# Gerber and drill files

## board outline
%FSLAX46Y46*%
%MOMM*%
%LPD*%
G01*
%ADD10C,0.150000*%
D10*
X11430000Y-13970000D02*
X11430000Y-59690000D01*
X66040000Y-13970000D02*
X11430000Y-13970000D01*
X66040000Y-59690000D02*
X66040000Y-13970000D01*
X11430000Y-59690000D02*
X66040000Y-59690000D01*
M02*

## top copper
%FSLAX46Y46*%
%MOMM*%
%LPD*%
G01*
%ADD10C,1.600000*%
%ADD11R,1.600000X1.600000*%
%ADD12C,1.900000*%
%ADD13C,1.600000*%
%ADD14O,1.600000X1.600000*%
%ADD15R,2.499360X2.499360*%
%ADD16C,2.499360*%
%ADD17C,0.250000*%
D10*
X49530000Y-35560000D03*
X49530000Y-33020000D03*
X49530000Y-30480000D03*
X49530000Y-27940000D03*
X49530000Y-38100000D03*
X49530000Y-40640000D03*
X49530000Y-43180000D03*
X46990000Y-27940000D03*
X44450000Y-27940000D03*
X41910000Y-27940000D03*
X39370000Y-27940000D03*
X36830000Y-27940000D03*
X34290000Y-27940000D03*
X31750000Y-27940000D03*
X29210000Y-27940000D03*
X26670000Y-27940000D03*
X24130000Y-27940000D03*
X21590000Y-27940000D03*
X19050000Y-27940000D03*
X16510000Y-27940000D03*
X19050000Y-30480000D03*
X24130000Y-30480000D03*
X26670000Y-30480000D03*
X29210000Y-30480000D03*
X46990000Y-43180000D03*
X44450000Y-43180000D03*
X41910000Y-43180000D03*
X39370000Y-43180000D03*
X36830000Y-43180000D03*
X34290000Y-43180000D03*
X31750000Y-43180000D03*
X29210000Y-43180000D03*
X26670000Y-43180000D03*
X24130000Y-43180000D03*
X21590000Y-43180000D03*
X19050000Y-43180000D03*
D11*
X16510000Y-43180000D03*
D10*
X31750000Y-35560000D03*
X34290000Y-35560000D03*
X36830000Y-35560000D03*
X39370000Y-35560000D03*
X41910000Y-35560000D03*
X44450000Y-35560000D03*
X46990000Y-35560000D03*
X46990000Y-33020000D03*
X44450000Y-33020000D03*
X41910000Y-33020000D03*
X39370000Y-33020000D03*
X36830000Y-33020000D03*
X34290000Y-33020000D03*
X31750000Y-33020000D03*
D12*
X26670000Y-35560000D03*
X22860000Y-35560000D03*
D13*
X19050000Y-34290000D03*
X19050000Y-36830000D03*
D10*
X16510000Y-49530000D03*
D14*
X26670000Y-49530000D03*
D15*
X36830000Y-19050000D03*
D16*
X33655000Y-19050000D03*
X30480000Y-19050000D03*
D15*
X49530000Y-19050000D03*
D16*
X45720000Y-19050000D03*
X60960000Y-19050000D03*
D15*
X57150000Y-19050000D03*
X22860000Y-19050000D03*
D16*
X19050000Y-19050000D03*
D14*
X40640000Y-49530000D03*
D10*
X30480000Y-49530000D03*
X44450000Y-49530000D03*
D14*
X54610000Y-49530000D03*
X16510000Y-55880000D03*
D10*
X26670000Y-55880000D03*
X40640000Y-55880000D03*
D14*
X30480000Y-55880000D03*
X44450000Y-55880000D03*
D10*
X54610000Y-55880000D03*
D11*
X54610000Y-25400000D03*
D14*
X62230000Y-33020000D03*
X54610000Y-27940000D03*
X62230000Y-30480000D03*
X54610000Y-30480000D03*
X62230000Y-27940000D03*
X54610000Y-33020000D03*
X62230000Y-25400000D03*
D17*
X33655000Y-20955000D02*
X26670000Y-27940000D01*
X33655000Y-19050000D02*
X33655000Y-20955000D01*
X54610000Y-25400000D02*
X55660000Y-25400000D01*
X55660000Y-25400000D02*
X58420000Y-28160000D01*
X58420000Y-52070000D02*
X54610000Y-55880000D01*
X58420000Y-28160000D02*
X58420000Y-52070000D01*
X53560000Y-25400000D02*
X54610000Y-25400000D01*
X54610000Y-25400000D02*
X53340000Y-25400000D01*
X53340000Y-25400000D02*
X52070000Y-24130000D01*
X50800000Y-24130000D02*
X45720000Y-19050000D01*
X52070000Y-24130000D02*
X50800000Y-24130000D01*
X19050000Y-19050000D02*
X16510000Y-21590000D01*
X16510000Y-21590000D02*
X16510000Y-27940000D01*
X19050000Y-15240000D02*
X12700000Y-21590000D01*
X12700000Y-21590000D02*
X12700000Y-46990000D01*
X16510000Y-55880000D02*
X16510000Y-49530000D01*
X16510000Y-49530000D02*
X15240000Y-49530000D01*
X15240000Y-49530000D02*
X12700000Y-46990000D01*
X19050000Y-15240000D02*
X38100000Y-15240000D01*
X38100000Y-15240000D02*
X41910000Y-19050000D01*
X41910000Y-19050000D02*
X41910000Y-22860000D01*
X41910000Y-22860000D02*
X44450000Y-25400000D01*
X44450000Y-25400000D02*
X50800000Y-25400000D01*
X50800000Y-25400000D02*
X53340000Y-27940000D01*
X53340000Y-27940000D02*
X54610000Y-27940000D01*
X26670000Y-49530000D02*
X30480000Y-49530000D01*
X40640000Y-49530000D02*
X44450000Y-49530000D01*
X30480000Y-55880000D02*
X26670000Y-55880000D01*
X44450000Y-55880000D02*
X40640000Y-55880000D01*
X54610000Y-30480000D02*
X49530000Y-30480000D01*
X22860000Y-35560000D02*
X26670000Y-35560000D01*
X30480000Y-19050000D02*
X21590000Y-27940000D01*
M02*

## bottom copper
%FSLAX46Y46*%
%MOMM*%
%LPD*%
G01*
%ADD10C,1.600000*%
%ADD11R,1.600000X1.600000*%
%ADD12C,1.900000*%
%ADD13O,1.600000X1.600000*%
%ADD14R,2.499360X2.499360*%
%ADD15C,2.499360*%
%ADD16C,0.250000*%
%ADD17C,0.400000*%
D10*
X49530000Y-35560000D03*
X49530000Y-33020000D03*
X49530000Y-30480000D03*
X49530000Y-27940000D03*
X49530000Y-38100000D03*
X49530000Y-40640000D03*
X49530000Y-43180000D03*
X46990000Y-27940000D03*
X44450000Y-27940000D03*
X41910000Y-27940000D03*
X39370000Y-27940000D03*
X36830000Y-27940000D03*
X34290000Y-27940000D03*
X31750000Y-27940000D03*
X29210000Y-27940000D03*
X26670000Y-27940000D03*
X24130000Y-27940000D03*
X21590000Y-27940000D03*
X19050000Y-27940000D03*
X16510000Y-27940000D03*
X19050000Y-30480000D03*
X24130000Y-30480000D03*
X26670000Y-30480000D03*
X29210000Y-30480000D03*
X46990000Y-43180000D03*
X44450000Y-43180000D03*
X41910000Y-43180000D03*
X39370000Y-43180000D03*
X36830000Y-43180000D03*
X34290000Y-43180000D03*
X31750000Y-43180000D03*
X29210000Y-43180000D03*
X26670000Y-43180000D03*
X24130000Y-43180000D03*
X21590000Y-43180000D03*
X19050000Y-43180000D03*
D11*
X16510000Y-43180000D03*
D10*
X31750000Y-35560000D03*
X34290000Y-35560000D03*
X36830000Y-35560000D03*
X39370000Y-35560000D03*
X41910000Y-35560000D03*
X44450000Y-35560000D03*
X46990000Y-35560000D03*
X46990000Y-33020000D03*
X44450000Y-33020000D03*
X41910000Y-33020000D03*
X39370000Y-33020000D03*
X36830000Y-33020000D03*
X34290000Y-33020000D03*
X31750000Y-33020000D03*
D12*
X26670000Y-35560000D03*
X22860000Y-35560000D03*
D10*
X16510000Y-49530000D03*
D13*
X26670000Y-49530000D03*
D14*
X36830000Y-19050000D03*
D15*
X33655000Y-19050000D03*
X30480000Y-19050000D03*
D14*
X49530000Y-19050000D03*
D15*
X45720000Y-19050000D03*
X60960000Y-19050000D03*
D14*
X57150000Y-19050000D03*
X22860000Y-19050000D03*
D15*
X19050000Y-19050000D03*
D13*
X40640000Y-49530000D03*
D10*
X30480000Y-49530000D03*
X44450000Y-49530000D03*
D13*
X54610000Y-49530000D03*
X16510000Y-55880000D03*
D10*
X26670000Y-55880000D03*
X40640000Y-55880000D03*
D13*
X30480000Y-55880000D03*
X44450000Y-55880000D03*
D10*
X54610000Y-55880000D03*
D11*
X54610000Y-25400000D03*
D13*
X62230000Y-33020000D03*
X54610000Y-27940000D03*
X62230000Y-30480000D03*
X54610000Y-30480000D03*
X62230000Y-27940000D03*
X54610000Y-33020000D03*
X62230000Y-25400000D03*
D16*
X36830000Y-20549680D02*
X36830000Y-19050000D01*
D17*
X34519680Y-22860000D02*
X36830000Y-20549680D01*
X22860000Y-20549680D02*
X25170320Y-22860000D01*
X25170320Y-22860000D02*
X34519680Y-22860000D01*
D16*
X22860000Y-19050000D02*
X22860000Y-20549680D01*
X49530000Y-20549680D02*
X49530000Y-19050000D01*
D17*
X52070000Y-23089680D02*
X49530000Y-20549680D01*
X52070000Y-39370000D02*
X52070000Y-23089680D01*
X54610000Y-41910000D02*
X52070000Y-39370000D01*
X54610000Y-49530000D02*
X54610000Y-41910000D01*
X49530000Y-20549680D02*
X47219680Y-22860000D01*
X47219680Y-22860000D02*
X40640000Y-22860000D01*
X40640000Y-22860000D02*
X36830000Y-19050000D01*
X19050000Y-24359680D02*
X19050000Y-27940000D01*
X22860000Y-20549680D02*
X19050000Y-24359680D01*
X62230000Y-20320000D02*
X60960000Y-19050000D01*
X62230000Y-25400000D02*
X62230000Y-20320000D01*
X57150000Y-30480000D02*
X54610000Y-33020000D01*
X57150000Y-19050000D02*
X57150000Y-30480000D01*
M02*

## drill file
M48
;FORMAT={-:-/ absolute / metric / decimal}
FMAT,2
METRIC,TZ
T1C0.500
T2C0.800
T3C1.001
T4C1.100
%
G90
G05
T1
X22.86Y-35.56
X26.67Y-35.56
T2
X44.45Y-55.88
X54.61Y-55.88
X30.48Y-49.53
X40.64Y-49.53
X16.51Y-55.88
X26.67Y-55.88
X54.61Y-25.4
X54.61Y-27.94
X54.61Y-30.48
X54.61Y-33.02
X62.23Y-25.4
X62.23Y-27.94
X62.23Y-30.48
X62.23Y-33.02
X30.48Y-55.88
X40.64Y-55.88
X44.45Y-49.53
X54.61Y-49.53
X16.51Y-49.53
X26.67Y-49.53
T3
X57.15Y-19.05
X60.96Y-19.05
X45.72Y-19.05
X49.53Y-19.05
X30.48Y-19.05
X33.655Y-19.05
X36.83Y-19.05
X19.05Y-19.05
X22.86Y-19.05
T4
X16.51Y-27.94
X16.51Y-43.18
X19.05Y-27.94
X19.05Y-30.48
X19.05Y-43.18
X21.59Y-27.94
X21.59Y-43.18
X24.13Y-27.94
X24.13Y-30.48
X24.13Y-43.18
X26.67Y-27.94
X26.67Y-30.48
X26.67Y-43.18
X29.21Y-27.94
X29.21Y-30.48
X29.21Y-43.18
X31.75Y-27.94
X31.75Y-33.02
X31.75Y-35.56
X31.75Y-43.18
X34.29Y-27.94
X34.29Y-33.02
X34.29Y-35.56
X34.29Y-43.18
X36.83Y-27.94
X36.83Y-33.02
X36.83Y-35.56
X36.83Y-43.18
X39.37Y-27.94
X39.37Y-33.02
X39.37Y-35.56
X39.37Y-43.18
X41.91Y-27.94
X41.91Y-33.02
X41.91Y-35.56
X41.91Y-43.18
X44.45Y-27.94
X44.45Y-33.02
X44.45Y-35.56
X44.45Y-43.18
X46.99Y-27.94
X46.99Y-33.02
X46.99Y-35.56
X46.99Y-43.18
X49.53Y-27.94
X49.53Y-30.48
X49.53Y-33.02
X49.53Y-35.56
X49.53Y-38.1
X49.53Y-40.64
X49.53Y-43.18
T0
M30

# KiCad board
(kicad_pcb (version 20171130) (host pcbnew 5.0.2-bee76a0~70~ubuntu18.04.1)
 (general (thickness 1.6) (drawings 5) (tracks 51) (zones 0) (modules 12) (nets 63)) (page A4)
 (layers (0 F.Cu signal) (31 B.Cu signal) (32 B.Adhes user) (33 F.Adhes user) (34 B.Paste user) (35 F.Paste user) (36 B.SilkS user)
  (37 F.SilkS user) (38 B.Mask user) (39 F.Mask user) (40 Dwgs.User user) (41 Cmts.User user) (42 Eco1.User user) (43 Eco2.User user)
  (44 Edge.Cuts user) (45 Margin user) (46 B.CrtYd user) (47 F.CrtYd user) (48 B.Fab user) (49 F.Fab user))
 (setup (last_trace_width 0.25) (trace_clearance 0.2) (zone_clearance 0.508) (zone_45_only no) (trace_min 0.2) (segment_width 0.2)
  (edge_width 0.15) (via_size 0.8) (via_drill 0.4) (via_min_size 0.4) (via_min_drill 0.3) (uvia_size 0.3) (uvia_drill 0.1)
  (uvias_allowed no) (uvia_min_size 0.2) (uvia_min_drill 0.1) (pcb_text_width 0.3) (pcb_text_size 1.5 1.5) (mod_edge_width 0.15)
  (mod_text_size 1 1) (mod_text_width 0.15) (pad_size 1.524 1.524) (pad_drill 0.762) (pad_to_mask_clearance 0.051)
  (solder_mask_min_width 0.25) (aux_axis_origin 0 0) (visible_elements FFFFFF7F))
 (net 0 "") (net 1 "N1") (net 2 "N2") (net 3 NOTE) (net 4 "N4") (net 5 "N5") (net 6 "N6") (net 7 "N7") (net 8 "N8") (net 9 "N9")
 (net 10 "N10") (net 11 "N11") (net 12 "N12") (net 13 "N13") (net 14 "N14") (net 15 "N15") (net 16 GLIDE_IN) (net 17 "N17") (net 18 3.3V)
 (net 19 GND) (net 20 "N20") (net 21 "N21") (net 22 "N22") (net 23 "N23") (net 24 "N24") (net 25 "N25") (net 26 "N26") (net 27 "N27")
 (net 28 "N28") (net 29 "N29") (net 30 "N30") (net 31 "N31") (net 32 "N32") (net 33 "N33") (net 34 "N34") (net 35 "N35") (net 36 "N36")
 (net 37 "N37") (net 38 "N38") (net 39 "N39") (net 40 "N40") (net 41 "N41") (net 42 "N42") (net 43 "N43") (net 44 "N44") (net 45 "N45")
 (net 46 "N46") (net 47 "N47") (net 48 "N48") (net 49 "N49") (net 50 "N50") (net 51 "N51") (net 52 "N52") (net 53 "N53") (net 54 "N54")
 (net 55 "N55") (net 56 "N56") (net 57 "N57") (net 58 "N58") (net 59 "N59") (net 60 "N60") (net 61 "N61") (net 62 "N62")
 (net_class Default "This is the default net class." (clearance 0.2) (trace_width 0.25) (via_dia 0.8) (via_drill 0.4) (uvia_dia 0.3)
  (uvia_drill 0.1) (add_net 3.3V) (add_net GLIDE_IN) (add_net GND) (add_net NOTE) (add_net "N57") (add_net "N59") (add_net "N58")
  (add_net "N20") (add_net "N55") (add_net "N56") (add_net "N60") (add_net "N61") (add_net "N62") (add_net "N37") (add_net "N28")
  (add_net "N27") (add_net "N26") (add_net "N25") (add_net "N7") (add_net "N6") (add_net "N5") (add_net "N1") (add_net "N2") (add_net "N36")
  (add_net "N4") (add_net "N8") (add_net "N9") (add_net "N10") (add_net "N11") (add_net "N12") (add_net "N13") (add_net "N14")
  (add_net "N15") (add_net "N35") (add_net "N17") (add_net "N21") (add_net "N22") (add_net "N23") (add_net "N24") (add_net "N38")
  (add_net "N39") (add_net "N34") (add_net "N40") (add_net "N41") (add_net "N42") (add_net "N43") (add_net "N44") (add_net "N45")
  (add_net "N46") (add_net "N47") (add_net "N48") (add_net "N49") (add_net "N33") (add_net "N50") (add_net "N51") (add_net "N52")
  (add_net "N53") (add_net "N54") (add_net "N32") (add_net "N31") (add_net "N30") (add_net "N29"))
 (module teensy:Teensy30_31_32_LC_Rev (layer F.Cu) (at 33.02 35.56)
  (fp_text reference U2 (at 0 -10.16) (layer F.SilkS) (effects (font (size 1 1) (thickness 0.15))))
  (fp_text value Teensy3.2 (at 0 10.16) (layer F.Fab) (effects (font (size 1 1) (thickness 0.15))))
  (pad 17 thru_hole circle (at 16.51 0) (size 1.6 1.6) (drill 1.1) (layers *.Cu *.Mask F.SilkS) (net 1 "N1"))
  (pad 18 thru_hole circle (at 16.51 -2.54) (size 1.6 1.6) (drill 1.1) (layers *.Cu *.Mask F.SilkS) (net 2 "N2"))
  (pad 19 thru_hole circle (at 16.51 -5.08) (size 1.6 1.6) (drill 1.1) (layers *.Cu *.Mask F.SilkS) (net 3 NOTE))
  (pad 20 thru_hole circle (at 16.51 -7.62) (size 1.6 1.6) (drill 1.1) (layers *.Cu *.Mask F.SilkS) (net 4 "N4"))
  (pad 16 thru_hole circle (at 16.51 2.54) (size 1.6 1.6) (drill 1.1) (layers *.Cu *.Mask F.SilkS) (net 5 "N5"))
  (pad 15 thru_hole circle (at 16.51 5.08) (size 1.6 1.6) (drill 1.1) (layers *.Cu *.Mask F.SilkS) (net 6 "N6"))
  (pad 14 thru_hole circle (at 16.51 7.62) (size 1.6 1.6) (drill 1.1) (layers *.Cu *.Mask F.SilkS) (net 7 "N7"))
  (pad 21 thru_hole circle (at 13.97 -7.62) (size 1.6 1.6) (drill 1.1) (layers *.Cu *.Mask F.SilkS) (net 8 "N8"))
  (pad 22 thru_hole circle (at 11.43 -7.62) (size 1.6 1.6) (drill 1.1) (layers *.Cu *.Mask F.SilkS) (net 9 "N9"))
  (pad 23 thru_hole circle (at 8.89 -7.62) (size 1.6 1.6) (drill 1.1) (layers *.Cu *.Mask F.SilkS) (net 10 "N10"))
  (pad 24 thru_hole circle (at 6.35 -7.62) (size 1.6 1.6) (drill 1.1) (layers *.Cu *.Mask F.SilkS) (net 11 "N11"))
  (pad 25 thru_hole circle (at 3.81 -7.62) (size 1.6 1.6) (drill 1.1) (layers *.Cu *.Mask F.SilkS) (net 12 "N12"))
  (pad 26 thru_hole circle (at 1.27 -7.62) (size 1.6 1.6) (drill 1.1) (layers *.Cu *.Mask F.SilkS) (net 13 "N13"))
  (pad 27 thru_hole circle (at -1.27 -7.62) (size 1.6 1.6) (drill 1.1) (layers *.Cu *.Mask F.SilkS) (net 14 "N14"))
  (pad 28 thru_hole circle (at -3.81 -7.62) (size 1.6 1.6) (drill 1.1) (layers *.Cu *.Mask F.SilkS) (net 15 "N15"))
  (pad 29 thru_hole circle (at -6.35 -7.62) (size 1.6 1.6) (drill 1.1) (layers *.Cu *.Mask F.SilkS) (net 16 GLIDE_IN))
  (pad 30 thru_hole circle (at -8.89 -7.62) (size 1.6 1.6) (drill 1.1) (layers *.Cu *.Mask F.SilkS) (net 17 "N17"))
  (pad 31 thru_hole circle (at -11.43 -7.62) (size 1.6 1.6) (drill 1.1) (layers *.Cu *.Mask F.SilkS) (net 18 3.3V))
  (pad 32 thru_hole circle (at -13.97 -7.62) (size 1.6 1.6) (drill 1.1) (layers *.Cu *.Mask F.SilkS) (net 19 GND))
  (pad 33 thru_hole circle (at -16.51 -7.62) (size 1.6 1.6) (drill 1.1) (layers *.Cu *.Mask F.SilkS) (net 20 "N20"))
  (pad 34 thru_hole circle (at -13.97 -5.08) (size 1.6 1.6) (drill 1.1) (layers *.Cu *.Mask F.SilkS) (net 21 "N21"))
  (pad 35 thru_hole circle (at -8.89 -5.08) (size 1.6 1.6) (drill 1.1) (layers *.Cu *.Mask F.SilkS) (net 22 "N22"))
  (pad 36 thru_hole circle (at -6.35 -5.08) (size 1.6 1.6) (drill 1.1) (layers *.Cu *.Mask F.SilkS) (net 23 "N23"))
  (pad 37 thru_hole circle (at -3.81 -5.08) (size 1.6 1.6) (drill 1.1) (layers *.Cu *.Mask F.SilkS) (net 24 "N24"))
  (pad 13 thru_hole circle (at 13.97 7.62) (size 1.6 1.6) (drill 1.1) (layers *.Cu *.Mask F.SilkS) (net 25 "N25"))
  (pad 12 thru_hole circle (at 11.43 7.62) (size 1.6 1.6) (drill 1.1) (layers *.Cu *.Mask F.SilkS) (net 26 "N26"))
  (pad 11 thru_hole circle (at 8.89 7.62) (size 1.6 1.6) (drill 1.1) (layers *.Cu *.Mask F.SilkS) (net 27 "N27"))
  (pad 10 thru_hole circle (at 6.35 7.62) (size 1.6 1.6) (drill 1.1) (layers *.Cu *.Mask F.SilkS) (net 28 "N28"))
  (pad 9 thru_hole circle (at 3.81 7.62) (size 1.6 1.6) (drill 1.1) (layers *.Cu *.Mask F.SilkS) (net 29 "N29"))
  (pad 8 thru_hole circle (at 1.27 7.62) (size 1.6 1.6) (drill 1.1) (layers *.Cu *.Mask F.SilkS) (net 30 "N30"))
  (pad 7 thru_hole circle (at -1.27 7.62) (size 1.6 1.6) (drill 1.1) (layers *.Cu *.Mask F.SilkS) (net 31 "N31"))
  (pad 6 thru_hole circle (at -3.81 7.62) (size 1.6 1.6) (drill 1.1) (layers *.Cu *.Mask F.SilkS) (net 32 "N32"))
  (pad 5 thru_hole circle (at -6.35 7.62) (size 1.6 1.6) (drill 1.1) (layers *.Cu *.Mask F.SilkS) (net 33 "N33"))
  (pad 4 thru_hole circle (at -8.89 7.62) (size 1.6 1.6) (drill 1.1) (layers *.Cu *.Mask F.SilkS) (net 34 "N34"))
  (pad 3 thru_hole circle (at -11.43 7.62) (size 1.6 1.6) (drill 1.1) (layers *.Cu *.Mask F.SilkS) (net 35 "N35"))
  (pad 2 thru_hole circle (at -13.97 7.62) (size 1.6 1.6) (drill 1.1) (layers *.Cu *.Mask F.SilkS) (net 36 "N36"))
  (pad 1 thru_hole rect (at -16.51 7.62) (size 1.6 1.6) (drill 1.1) (layers *.Cu *.Mask F.SilkS) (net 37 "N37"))
  (pad 38 thru_hole circle (at -1.27 0) (size 1.6 1.6) (drill 1.1) (layers *.Cu *.Mask) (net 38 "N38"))
  (pad 39 thru_hole circle (at 1.27 0) (size 1.6 1.6) (drill 1.1) (layers *.Cu *.Mask) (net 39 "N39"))
  (pad 40 thru_hole circle (at 3.81 0) (size 1.6 1.6) (drill 1.1) (layers *.Cu *.Mask) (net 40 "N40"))
  (pad 41 thru_hole circle (at 6.35 0) (size 1.6 1.6) (drill 1.1) (layers *.Cu *.Mask) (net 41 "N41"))
  (pad 42 thru_hole circle (at 8.89 0) (size 1.6 1.6) (drill 1.1) (layers *.Cu *.Mask) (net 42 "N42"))
  (pad 43 thru_hole circle (at 11.43 0) (size 1.6 1.6) (drill 1.1) (layers *.Cu *.Mask) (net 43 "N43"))
  (pad 44 thru_hole circle (at 13.97 0) (size 1.6 1.6) (drill 1.1) (layers *.Cu *.Mask) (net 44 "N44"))
  (pad 45 thru_hole circle (at 13.97 -2.54) (size 1.6 1.6) (drill 1.1) (layers *.Cu *.Mask) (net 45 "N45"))
  (pad 46 thru_hole circle (at 11.43 -2.54) (size 1.6 1.6) (drill 1.1) (layers *.Cu *.Mask) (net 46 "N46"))
  (pad 47 thru_hole circle (at 8.89 -2.54) (size 1.6 1.6) (drill 1.1) (layers *.Cu *.Mask) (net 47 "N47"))
  (pad 48 thru_hole circle (at 6.35 -2.54) (size 1.6 1.6) (drill 1.1) (layers *.Cu *.Mask) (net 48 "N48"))
  (pad 49 thru_hole circle (at 3.81 -2.54) (size 1.6 1.6) (drill 1.1) (layers *.Cu *.Mask) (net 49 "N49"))
  (pad 50 thru_hole circle (at 1.27 -2.54) (size 1.6 1.6) (drill 1.1) (layers *.Cu *.Mask) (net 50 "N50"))
  (pad 51 thru_hole circle (at -1.27 -2.54) (size 1.6 1.6) (drill 1.1) (layers *.Cu *.Mask) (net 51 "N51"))
  (pad 52 thru_hole circle (at -6.35 0) (size 1.9 1.9) (drill 0.5) (layers *.Cu *.Mask F.SilkS) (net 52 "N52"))
  (pad 52 thru_hole circle (at -10.16 0) (size 1.9 1.9) (drill 0.5) (layers *.Cu *.Mask F.SilkS) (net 52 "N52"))
  (pad 53 smd circle (at -13.97 -1.27) (size 1.6 1.6) (layers F.Cu F.Paste F.Mask) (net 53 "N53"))
  (pad 54 smd circle (at -13.97 1.27) (size 1.6 1.6) (layers F.Cu F.Paste F.Mask) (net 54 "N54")))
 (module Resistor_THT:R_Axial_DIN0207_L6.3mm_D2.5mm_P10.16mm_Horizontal (layer F.Cu) (at 16.51 49.53)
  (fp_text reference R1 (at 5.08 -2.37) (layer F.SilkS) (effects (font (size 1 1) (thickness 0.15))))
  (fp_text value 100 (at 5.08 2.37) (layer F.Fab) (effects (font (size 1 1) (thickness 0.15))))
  (pad 1 thru_hole circle (at 0 0) (size 1.6 1.6) (drill 0.8) (layers *.Cu *.Mask) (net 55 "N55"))
  (pad 2 thru_hole oval (at 10.16 0) (size 1.6 1.6) (drill 0.8) (layers *.Cu *.Mask) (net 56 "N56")))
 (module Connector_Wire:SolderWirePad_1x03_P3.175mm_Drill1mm (layer F.Cu) (at 36.83 19.05 180)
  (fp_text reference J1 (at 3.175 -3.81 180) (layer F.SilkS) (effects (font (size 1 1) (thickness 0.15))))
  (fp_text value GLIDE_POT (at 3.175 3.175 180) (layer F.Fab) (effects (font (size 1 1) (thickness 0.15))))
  (pad 1 thru_hole rect (at 0 0 180) (size 2.49936 2.49936) (drill 1.00076) (layers *.Cu *.Mask) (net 19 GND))
  (pad 2 thru_hole circle (at 3.175 0 180) (size 2.49936 2.49936) (drill 1.00076) (layers *.Cu *.Mask) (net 16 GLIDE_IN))
  (pad 3 thru_hole circle (at 6.35 0 180) (size 2.49936 2.49936) (drill 1.00076) (layers *.Cu *.Mask) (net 18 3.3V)))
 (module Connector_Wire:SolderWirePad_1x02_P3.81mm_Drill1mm (layer F.Cu) (at 49.53 19.05 180)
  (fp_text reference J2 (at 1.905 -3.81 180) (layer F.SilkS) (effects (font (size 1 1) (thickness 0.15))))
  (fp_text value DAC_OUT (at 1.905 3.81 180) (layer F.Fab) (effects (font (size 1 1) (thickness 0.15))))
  (pad 1 thru_hole rect (at 0 0 180) (size 2.49936 2.49936) (drill 1.00076) (layers *.Cu *.Mask) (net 19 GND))
  (pad 2 thru_hole circle (at 3.81 0 180) (size 2.49936 2.49936) (drill 1.00076) (layers *.Cu *.Mask) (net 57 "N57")))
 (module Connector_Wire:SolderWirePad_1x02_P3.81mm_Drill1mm (layer F.Cu) (at 57.15 19.05)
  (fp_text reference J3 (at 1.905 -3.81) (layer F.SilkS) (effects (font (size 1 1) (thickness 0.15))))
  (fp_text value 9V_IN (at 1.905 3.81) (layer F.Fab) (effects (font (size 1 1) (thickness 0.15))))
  (pad 2 thru_hole circle (at 3.81 0) (size 2.49936 2.49936) (drill 1.00076) (layers *.Cu *.Mask) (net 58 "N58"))
  (pad 1 thru_hole rect (at 0 0) (size 2.49936 2.49936) (drill 1.00076) (layers *.Cu *.Mask) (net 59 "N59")))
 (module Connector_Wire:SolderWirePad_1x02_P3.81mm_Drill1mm (layer F.Cu) (at 22.86 19.05 180)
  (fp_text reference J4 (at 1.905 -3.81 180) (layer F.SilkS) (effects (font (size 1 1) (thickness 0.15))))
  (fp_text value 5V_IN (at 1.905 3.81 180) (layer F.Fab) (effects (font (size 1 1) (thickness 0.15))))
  (pad 1 thru_hole rect (at 0 0 180) (size 2.49936 2.49936) (drill 1.00076) (layers *.Cu *.Mask) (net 19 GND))
  (pad 2 thru_hole circle (at 3.81 0 180) (size 2.49936 2.49936) (drill 1.00076) (layers *.Cu *.Mask) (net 20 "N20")))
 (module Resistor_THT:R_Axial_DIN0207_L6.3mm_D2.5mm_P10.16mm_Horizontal (layer F.Cu) (at 30.48 49.53)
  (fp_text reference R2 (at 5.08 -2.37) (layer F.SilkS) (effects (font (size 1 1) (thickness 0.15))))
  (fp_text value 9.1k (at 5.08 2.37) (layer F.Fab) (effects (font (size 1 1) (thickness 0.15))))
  (pad 2 thru_hole oval (at 10.16 0) (size 1.6 1.6) (drill 0.8) (layers *.Cu *.Mask) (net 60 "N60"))
  (pad 1 thru_hole circle (at 0 0) (size 1.6 1.6) (drill 0.8) (layers *.Cu *.Mask) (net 56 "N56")))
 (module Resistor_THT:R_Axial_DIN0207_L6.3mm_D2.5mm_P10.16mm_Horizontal (layer F.Cu) (at 44.45 49.53)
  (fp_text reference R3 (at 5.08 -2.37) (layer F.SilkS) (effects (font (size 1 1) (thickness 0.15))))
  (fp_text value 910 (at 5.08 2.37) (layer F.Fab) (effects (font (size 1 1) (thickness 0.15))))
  (pad 1 thru_hole circle (at 0 0) (size 1.6 1.6) (drill 0.8) (layers *.Cu *.Mask) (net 60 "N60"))
  (pad 2 thru_hole oval (at 10.16 0) (size 1.6 1.6) (drill 0.8) (layers *.Cu *.Mask) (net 19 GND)))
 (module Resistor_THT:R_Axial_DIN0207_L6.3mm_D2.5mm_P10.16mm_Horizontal (layer F.Cu) (at 26.67 55.88 180)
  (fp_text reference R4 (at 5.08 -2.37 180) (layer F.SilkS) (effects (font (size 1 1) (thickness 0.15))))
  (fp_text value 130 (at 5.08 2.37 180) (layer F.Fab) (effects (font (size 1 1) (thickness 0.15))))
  (pad 2 thru_hole oval (at 10.16 0 180) (size 1.6 1.6) (drill 0.8) (layers *.Cu *.Mask) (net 55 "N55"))
  (pad 1 thru_hole circle (at 0 0 180) (size 1.6 1.6) (drill 0.8) (layers *.Cu *.Mask) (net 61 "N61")))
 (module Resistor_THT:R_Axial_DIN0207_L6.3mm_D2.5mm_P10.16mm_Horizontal (layer F.Cu) (at 40.64 55.88 180)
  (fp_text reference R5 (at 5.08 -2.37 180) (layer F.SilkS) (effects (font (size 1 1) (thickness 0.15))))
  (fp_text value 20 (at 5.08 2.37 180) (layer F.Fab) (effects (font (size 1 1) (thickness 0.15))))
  (pad 1 thru_hole circle (at 0 0 180) (size 1.6 1.6) (drill 0.8) (layers *.Cu *.Mask) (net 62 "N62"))
  (pad 2 thru_hole oval (at 10.16 0 180) (size 1.6 1.6) (drill 0.8) (layers *.Cu *.Mask) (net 61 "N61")))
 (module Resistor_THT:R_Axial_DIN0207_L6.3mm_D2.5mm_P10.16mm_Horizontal (layer F.Cu) (at 54.61 55.88 180)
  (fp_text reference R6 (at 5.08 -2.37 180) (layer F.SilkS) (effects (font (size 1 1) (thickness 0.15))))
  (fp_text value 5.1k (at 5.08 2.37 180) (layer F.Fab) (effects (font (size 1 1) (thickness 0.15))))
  (pad 2 thru_hole oval (at 10.16 0 180) (size 1.6 1.6) (drill 0.8) (layers *.Cu *.Mask) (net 62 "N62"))
  (pad 1 thru_hole circle (at 0 0 180) (size 1.6 1.6) (drill 0.8) (layers *.Cu *.Mask) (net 57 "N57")))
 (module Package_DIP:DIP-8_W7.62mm (layer F.Cu) (at 54.61 25.4)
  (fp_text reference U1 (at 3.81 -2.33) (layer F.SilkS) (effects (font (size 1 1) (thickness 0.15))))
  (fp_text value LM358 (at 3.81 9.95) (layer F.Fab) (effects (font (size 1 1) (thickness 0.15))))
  (pad 1 thru_hole rect (at 0 0) (size 1.6 1.6) (drill 0.8) (layers *.Cu *.Mask) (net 57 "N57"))
  (pad 5 thru_hole oval (at 7.62 7.62) (size 1.6 1.6) (drill 0.8) (layers *.Cu *.Mask))
  (pad 2 thru_hole oval (at 0 2.54) (size 1.6 1.6) (drill 0.8) (layers *.Cu *.Mask) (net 55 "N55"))
  (pad 6 thru_hole oval (at 7.62 5.08) (size 1.6 1.6) (drill 0.8) (layers *.Cu *.Mask))
  (pad 3 thru_hole oval (at 0 5.08) (size 1.6 1.6) (drill 0.8) (layers *.Cu *.Mask) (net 3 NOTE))
  (pad 7 thru_hole oval (at 7.62 2.54) (size 1.6 1.6) (drill 0.8) (layers *.Cu *.Mask))
  (pad 4 thru_hole oval (at 0 7.62) (size 1.6 1.6) (drill 0.8) (layers *.Cu *.Mask) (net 59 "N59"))
  (pad 8 thru_hole oval (at 7.62 0) (size 1.6 1.6) (drill 0.8) (layers *.Cu *.Mask) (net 58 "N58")))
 (gr_line (start 11.43 13.97) (end 11.43 59.69) (layer Edge.Cuts) (width 0.15))
 (gr_line (start 66.04 13.97) (end 11.43 13.97) (layer Edge.Cuts) (width 0.15))
 (gr_line (start 66.04 59.69) (end 66.04 13.97) (layer Edge.Cuts) (width 0.15))
 (gr_line (start 11.43 59.69) (end 66.04 59.69) (layer Edge.Cuts) (width 0.15))
 (segment (start 36.83 20.54968) (end 36.83 19.05) (width 0.25) (layer B.Cu) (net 19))
 (segment (start 34.51968 22.86) (end 36.83 20.54968) (width 0.4) (layer B.Cu) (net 19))
 (segment (start 22.86 20.54968) (end 25.17032 22.86) (width 0.4) (layer B.Cu) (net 19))
 (segment (start 25.17032 22.86) (end 34.51968 22.86) (width 0.4) (layer B.Cu) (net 19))
 (segment (start 22.86 19.05) (end 22.86 20.54968) (width 0.25) (layer B.Cu) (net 19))
 (segment (start 49.53 20.54968) (end 49.53 19.05) (width 0.25) (layer B.Cu) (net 19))
 (segment (start 52.07 23.08968) (end 49.53 20.54968) (width 0.4) (layer B.Cu) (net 19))
 (segment (start 52.07 39.37) (end 52.07 23.08968) (width 0.4) (layer B.Cu) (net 19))
 (segment (start 54.61 41.91) (end 52.07 39.37) (width 0.4) (layer B.Cu) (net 19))
 (segment (start 54.61 49.53) (end 54.61 41.91) (width 0.4) (layer B.Cu) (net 19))
 (segment (start 49.53 20.54968) (end 47.21968 22.86) (width 0.4) (layer B.Cu) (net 19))
 (segment (start 47.21968 22.86) (end 40.64 22.86) (width 0.4) (layer B.Cu) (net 19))
 (segment (start 40.64 22.86) (end 36.83 19.05) (width 0.4) (layer B.Cu) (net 19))
 (segment (start 19.05 24.35968) (end 19.05 27.94) (width 0.4) (layer B.Cu) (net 19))
 (segment (start 22.86 20.54968) (end 19.05 24.35968) (width 0.4) (layer B.Cu) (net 19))
 (segment (start 33.655 20.955) (end 26.67 27.94) (width 0.25) (layer F.Cu) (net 16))
 (segment (start 33.655 19.05) (end 33.655 20.955) (width 0.25) (layer F.Cu) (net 16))
 (segment (start 54.61 25.4) (end 55.66 25.4) (width 0.25) (layer F.Cu) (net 57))
 (segment (start 55.66 25.4) (end 58.42 28.16) (width 0.25) (layer F.Cu) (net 57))
 (segment (start 58.42 52.07) (end 54.61 55.88) (width 0.25) (layer F.Cu) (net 57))
 (segment (start 58.42 28.16) (end 58.42 52.07) (width 0.25) (layer F.Cu) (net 57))
 (segment (start 53.56 25.4) (end 54.61 25.4) (width 0.25) (layer F.Cu) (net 57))
 (segment (start 54.61 25.4) (end 53.34 25.4) (width 0.25) (layer F.Cu) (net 57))
 (segment (start 53.34 25.4) (end 52.07 24.13) (width 0.25) (layer F.Cu) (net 57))
 (segment (start 50.8 24.13) (end 45.72 19.05) (width 0.25) (layer F.Cu) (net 57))
 (segment (start 52.07 24.13) (end 50.8 24.13) (width 0.25) (layer F.Cu) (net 57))
 (segment (start 62.23 20.32) (end 60.96 19.05) (width 0.4) (layer B.Cu) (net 58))
 (segment (start 62.23 25.4) (end 62.23 20.32) (width 0.4) (layer B.Cu) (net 58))
 (segment (start 57.15 30.48) (end 54.61 33.02) (width 0.4) (layer B.Cu) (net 59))
 (segment (start 57.15 19.05) (end 57.15 30.48) (width 0.4) (layer B.Cu) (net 59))
 (segment (start 19.05 19.05) (end 16.51 21.59) (width 0.25) (layer F.Cu) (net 20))
 (segment (start 16.51 21.59) (end 16.51 27.94) (width 0.25) (layer F.Cu) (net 20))
 (segment (start 19.05 15.24) (end 12.7 21.59) (width 0.25) (layer F.Cu) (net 55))
 (segment (start 12.7 21.59) (end 12.7 46.99) (width 0.25) (layer F.Cu) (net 55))
 (segment (start 16.51 55.88) (end 16.51 49.53) (width 0.25) (layer F.Cu) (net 55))
 (segment (start 16.51 49.53) (end 15.24 49.53) (width 0.25) (layer F.Cu) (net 55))
 (segment (start 15.24 49.53) (end 12.7 46.99) (width 0.25) (layer F.Cu) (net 55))
 (segment (start 19.05 15.24) (end 38.1 15.24) (width 0.25) (layer F.Cu) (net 55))
 (segment (start 38.1 15.24) (end 41.91 19.05) (width 0.25) (layer F.Cu) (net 55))
 (segment (start 41.91 19.05) (end 41.91 22.86) (width 0.25) (layer F.Cu) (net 55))
 (segment (start 41.91 22.86) (end 44.45 25.4) (width 0.25) (layer F.Cu) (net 55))
 (segment (start 44.45 25.4) (end 50.8 25.4) (width 0.25) (layer F.Cu) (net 55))
 (segment (start 50.8 25.4) (end 53.34 27.94) (width 0.25) (layer F.Cu) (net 55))
 (segment (start 53.34 27.94) (end 54.61 27.94) (width 0.25) (layer F.Cu) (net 55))
 (segment (start 26.67 49.53) (end 30.48 49.53) (width 0.25) (layer F.Cu) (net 56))
 (segment (start 40.64 49.53) (end 44.45 49.53) (width 0.25) (layer F.Cu) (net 60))
 (segment (start 30.48 55.88) (end 26.67 55.88) (width 0.25) (layer F.Cu) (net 61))
 (segment (start 44.45 55.88) (end 40.64 55.88) (width 0.25) (layer F.Cu) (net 62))
 (segment (start 54.61 30.48) (end 49.53 30.48) (width 0.25) (layer F.Cu) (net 3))
 (segment (start 22.86 35.56) (end 26.67 35.56) (width 0.25) (layer F.Cu) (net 52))
 (segment (start 30.48 19.05) (end 21.59 27.94) (width 0.25) (layer F.Cu) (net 18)))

